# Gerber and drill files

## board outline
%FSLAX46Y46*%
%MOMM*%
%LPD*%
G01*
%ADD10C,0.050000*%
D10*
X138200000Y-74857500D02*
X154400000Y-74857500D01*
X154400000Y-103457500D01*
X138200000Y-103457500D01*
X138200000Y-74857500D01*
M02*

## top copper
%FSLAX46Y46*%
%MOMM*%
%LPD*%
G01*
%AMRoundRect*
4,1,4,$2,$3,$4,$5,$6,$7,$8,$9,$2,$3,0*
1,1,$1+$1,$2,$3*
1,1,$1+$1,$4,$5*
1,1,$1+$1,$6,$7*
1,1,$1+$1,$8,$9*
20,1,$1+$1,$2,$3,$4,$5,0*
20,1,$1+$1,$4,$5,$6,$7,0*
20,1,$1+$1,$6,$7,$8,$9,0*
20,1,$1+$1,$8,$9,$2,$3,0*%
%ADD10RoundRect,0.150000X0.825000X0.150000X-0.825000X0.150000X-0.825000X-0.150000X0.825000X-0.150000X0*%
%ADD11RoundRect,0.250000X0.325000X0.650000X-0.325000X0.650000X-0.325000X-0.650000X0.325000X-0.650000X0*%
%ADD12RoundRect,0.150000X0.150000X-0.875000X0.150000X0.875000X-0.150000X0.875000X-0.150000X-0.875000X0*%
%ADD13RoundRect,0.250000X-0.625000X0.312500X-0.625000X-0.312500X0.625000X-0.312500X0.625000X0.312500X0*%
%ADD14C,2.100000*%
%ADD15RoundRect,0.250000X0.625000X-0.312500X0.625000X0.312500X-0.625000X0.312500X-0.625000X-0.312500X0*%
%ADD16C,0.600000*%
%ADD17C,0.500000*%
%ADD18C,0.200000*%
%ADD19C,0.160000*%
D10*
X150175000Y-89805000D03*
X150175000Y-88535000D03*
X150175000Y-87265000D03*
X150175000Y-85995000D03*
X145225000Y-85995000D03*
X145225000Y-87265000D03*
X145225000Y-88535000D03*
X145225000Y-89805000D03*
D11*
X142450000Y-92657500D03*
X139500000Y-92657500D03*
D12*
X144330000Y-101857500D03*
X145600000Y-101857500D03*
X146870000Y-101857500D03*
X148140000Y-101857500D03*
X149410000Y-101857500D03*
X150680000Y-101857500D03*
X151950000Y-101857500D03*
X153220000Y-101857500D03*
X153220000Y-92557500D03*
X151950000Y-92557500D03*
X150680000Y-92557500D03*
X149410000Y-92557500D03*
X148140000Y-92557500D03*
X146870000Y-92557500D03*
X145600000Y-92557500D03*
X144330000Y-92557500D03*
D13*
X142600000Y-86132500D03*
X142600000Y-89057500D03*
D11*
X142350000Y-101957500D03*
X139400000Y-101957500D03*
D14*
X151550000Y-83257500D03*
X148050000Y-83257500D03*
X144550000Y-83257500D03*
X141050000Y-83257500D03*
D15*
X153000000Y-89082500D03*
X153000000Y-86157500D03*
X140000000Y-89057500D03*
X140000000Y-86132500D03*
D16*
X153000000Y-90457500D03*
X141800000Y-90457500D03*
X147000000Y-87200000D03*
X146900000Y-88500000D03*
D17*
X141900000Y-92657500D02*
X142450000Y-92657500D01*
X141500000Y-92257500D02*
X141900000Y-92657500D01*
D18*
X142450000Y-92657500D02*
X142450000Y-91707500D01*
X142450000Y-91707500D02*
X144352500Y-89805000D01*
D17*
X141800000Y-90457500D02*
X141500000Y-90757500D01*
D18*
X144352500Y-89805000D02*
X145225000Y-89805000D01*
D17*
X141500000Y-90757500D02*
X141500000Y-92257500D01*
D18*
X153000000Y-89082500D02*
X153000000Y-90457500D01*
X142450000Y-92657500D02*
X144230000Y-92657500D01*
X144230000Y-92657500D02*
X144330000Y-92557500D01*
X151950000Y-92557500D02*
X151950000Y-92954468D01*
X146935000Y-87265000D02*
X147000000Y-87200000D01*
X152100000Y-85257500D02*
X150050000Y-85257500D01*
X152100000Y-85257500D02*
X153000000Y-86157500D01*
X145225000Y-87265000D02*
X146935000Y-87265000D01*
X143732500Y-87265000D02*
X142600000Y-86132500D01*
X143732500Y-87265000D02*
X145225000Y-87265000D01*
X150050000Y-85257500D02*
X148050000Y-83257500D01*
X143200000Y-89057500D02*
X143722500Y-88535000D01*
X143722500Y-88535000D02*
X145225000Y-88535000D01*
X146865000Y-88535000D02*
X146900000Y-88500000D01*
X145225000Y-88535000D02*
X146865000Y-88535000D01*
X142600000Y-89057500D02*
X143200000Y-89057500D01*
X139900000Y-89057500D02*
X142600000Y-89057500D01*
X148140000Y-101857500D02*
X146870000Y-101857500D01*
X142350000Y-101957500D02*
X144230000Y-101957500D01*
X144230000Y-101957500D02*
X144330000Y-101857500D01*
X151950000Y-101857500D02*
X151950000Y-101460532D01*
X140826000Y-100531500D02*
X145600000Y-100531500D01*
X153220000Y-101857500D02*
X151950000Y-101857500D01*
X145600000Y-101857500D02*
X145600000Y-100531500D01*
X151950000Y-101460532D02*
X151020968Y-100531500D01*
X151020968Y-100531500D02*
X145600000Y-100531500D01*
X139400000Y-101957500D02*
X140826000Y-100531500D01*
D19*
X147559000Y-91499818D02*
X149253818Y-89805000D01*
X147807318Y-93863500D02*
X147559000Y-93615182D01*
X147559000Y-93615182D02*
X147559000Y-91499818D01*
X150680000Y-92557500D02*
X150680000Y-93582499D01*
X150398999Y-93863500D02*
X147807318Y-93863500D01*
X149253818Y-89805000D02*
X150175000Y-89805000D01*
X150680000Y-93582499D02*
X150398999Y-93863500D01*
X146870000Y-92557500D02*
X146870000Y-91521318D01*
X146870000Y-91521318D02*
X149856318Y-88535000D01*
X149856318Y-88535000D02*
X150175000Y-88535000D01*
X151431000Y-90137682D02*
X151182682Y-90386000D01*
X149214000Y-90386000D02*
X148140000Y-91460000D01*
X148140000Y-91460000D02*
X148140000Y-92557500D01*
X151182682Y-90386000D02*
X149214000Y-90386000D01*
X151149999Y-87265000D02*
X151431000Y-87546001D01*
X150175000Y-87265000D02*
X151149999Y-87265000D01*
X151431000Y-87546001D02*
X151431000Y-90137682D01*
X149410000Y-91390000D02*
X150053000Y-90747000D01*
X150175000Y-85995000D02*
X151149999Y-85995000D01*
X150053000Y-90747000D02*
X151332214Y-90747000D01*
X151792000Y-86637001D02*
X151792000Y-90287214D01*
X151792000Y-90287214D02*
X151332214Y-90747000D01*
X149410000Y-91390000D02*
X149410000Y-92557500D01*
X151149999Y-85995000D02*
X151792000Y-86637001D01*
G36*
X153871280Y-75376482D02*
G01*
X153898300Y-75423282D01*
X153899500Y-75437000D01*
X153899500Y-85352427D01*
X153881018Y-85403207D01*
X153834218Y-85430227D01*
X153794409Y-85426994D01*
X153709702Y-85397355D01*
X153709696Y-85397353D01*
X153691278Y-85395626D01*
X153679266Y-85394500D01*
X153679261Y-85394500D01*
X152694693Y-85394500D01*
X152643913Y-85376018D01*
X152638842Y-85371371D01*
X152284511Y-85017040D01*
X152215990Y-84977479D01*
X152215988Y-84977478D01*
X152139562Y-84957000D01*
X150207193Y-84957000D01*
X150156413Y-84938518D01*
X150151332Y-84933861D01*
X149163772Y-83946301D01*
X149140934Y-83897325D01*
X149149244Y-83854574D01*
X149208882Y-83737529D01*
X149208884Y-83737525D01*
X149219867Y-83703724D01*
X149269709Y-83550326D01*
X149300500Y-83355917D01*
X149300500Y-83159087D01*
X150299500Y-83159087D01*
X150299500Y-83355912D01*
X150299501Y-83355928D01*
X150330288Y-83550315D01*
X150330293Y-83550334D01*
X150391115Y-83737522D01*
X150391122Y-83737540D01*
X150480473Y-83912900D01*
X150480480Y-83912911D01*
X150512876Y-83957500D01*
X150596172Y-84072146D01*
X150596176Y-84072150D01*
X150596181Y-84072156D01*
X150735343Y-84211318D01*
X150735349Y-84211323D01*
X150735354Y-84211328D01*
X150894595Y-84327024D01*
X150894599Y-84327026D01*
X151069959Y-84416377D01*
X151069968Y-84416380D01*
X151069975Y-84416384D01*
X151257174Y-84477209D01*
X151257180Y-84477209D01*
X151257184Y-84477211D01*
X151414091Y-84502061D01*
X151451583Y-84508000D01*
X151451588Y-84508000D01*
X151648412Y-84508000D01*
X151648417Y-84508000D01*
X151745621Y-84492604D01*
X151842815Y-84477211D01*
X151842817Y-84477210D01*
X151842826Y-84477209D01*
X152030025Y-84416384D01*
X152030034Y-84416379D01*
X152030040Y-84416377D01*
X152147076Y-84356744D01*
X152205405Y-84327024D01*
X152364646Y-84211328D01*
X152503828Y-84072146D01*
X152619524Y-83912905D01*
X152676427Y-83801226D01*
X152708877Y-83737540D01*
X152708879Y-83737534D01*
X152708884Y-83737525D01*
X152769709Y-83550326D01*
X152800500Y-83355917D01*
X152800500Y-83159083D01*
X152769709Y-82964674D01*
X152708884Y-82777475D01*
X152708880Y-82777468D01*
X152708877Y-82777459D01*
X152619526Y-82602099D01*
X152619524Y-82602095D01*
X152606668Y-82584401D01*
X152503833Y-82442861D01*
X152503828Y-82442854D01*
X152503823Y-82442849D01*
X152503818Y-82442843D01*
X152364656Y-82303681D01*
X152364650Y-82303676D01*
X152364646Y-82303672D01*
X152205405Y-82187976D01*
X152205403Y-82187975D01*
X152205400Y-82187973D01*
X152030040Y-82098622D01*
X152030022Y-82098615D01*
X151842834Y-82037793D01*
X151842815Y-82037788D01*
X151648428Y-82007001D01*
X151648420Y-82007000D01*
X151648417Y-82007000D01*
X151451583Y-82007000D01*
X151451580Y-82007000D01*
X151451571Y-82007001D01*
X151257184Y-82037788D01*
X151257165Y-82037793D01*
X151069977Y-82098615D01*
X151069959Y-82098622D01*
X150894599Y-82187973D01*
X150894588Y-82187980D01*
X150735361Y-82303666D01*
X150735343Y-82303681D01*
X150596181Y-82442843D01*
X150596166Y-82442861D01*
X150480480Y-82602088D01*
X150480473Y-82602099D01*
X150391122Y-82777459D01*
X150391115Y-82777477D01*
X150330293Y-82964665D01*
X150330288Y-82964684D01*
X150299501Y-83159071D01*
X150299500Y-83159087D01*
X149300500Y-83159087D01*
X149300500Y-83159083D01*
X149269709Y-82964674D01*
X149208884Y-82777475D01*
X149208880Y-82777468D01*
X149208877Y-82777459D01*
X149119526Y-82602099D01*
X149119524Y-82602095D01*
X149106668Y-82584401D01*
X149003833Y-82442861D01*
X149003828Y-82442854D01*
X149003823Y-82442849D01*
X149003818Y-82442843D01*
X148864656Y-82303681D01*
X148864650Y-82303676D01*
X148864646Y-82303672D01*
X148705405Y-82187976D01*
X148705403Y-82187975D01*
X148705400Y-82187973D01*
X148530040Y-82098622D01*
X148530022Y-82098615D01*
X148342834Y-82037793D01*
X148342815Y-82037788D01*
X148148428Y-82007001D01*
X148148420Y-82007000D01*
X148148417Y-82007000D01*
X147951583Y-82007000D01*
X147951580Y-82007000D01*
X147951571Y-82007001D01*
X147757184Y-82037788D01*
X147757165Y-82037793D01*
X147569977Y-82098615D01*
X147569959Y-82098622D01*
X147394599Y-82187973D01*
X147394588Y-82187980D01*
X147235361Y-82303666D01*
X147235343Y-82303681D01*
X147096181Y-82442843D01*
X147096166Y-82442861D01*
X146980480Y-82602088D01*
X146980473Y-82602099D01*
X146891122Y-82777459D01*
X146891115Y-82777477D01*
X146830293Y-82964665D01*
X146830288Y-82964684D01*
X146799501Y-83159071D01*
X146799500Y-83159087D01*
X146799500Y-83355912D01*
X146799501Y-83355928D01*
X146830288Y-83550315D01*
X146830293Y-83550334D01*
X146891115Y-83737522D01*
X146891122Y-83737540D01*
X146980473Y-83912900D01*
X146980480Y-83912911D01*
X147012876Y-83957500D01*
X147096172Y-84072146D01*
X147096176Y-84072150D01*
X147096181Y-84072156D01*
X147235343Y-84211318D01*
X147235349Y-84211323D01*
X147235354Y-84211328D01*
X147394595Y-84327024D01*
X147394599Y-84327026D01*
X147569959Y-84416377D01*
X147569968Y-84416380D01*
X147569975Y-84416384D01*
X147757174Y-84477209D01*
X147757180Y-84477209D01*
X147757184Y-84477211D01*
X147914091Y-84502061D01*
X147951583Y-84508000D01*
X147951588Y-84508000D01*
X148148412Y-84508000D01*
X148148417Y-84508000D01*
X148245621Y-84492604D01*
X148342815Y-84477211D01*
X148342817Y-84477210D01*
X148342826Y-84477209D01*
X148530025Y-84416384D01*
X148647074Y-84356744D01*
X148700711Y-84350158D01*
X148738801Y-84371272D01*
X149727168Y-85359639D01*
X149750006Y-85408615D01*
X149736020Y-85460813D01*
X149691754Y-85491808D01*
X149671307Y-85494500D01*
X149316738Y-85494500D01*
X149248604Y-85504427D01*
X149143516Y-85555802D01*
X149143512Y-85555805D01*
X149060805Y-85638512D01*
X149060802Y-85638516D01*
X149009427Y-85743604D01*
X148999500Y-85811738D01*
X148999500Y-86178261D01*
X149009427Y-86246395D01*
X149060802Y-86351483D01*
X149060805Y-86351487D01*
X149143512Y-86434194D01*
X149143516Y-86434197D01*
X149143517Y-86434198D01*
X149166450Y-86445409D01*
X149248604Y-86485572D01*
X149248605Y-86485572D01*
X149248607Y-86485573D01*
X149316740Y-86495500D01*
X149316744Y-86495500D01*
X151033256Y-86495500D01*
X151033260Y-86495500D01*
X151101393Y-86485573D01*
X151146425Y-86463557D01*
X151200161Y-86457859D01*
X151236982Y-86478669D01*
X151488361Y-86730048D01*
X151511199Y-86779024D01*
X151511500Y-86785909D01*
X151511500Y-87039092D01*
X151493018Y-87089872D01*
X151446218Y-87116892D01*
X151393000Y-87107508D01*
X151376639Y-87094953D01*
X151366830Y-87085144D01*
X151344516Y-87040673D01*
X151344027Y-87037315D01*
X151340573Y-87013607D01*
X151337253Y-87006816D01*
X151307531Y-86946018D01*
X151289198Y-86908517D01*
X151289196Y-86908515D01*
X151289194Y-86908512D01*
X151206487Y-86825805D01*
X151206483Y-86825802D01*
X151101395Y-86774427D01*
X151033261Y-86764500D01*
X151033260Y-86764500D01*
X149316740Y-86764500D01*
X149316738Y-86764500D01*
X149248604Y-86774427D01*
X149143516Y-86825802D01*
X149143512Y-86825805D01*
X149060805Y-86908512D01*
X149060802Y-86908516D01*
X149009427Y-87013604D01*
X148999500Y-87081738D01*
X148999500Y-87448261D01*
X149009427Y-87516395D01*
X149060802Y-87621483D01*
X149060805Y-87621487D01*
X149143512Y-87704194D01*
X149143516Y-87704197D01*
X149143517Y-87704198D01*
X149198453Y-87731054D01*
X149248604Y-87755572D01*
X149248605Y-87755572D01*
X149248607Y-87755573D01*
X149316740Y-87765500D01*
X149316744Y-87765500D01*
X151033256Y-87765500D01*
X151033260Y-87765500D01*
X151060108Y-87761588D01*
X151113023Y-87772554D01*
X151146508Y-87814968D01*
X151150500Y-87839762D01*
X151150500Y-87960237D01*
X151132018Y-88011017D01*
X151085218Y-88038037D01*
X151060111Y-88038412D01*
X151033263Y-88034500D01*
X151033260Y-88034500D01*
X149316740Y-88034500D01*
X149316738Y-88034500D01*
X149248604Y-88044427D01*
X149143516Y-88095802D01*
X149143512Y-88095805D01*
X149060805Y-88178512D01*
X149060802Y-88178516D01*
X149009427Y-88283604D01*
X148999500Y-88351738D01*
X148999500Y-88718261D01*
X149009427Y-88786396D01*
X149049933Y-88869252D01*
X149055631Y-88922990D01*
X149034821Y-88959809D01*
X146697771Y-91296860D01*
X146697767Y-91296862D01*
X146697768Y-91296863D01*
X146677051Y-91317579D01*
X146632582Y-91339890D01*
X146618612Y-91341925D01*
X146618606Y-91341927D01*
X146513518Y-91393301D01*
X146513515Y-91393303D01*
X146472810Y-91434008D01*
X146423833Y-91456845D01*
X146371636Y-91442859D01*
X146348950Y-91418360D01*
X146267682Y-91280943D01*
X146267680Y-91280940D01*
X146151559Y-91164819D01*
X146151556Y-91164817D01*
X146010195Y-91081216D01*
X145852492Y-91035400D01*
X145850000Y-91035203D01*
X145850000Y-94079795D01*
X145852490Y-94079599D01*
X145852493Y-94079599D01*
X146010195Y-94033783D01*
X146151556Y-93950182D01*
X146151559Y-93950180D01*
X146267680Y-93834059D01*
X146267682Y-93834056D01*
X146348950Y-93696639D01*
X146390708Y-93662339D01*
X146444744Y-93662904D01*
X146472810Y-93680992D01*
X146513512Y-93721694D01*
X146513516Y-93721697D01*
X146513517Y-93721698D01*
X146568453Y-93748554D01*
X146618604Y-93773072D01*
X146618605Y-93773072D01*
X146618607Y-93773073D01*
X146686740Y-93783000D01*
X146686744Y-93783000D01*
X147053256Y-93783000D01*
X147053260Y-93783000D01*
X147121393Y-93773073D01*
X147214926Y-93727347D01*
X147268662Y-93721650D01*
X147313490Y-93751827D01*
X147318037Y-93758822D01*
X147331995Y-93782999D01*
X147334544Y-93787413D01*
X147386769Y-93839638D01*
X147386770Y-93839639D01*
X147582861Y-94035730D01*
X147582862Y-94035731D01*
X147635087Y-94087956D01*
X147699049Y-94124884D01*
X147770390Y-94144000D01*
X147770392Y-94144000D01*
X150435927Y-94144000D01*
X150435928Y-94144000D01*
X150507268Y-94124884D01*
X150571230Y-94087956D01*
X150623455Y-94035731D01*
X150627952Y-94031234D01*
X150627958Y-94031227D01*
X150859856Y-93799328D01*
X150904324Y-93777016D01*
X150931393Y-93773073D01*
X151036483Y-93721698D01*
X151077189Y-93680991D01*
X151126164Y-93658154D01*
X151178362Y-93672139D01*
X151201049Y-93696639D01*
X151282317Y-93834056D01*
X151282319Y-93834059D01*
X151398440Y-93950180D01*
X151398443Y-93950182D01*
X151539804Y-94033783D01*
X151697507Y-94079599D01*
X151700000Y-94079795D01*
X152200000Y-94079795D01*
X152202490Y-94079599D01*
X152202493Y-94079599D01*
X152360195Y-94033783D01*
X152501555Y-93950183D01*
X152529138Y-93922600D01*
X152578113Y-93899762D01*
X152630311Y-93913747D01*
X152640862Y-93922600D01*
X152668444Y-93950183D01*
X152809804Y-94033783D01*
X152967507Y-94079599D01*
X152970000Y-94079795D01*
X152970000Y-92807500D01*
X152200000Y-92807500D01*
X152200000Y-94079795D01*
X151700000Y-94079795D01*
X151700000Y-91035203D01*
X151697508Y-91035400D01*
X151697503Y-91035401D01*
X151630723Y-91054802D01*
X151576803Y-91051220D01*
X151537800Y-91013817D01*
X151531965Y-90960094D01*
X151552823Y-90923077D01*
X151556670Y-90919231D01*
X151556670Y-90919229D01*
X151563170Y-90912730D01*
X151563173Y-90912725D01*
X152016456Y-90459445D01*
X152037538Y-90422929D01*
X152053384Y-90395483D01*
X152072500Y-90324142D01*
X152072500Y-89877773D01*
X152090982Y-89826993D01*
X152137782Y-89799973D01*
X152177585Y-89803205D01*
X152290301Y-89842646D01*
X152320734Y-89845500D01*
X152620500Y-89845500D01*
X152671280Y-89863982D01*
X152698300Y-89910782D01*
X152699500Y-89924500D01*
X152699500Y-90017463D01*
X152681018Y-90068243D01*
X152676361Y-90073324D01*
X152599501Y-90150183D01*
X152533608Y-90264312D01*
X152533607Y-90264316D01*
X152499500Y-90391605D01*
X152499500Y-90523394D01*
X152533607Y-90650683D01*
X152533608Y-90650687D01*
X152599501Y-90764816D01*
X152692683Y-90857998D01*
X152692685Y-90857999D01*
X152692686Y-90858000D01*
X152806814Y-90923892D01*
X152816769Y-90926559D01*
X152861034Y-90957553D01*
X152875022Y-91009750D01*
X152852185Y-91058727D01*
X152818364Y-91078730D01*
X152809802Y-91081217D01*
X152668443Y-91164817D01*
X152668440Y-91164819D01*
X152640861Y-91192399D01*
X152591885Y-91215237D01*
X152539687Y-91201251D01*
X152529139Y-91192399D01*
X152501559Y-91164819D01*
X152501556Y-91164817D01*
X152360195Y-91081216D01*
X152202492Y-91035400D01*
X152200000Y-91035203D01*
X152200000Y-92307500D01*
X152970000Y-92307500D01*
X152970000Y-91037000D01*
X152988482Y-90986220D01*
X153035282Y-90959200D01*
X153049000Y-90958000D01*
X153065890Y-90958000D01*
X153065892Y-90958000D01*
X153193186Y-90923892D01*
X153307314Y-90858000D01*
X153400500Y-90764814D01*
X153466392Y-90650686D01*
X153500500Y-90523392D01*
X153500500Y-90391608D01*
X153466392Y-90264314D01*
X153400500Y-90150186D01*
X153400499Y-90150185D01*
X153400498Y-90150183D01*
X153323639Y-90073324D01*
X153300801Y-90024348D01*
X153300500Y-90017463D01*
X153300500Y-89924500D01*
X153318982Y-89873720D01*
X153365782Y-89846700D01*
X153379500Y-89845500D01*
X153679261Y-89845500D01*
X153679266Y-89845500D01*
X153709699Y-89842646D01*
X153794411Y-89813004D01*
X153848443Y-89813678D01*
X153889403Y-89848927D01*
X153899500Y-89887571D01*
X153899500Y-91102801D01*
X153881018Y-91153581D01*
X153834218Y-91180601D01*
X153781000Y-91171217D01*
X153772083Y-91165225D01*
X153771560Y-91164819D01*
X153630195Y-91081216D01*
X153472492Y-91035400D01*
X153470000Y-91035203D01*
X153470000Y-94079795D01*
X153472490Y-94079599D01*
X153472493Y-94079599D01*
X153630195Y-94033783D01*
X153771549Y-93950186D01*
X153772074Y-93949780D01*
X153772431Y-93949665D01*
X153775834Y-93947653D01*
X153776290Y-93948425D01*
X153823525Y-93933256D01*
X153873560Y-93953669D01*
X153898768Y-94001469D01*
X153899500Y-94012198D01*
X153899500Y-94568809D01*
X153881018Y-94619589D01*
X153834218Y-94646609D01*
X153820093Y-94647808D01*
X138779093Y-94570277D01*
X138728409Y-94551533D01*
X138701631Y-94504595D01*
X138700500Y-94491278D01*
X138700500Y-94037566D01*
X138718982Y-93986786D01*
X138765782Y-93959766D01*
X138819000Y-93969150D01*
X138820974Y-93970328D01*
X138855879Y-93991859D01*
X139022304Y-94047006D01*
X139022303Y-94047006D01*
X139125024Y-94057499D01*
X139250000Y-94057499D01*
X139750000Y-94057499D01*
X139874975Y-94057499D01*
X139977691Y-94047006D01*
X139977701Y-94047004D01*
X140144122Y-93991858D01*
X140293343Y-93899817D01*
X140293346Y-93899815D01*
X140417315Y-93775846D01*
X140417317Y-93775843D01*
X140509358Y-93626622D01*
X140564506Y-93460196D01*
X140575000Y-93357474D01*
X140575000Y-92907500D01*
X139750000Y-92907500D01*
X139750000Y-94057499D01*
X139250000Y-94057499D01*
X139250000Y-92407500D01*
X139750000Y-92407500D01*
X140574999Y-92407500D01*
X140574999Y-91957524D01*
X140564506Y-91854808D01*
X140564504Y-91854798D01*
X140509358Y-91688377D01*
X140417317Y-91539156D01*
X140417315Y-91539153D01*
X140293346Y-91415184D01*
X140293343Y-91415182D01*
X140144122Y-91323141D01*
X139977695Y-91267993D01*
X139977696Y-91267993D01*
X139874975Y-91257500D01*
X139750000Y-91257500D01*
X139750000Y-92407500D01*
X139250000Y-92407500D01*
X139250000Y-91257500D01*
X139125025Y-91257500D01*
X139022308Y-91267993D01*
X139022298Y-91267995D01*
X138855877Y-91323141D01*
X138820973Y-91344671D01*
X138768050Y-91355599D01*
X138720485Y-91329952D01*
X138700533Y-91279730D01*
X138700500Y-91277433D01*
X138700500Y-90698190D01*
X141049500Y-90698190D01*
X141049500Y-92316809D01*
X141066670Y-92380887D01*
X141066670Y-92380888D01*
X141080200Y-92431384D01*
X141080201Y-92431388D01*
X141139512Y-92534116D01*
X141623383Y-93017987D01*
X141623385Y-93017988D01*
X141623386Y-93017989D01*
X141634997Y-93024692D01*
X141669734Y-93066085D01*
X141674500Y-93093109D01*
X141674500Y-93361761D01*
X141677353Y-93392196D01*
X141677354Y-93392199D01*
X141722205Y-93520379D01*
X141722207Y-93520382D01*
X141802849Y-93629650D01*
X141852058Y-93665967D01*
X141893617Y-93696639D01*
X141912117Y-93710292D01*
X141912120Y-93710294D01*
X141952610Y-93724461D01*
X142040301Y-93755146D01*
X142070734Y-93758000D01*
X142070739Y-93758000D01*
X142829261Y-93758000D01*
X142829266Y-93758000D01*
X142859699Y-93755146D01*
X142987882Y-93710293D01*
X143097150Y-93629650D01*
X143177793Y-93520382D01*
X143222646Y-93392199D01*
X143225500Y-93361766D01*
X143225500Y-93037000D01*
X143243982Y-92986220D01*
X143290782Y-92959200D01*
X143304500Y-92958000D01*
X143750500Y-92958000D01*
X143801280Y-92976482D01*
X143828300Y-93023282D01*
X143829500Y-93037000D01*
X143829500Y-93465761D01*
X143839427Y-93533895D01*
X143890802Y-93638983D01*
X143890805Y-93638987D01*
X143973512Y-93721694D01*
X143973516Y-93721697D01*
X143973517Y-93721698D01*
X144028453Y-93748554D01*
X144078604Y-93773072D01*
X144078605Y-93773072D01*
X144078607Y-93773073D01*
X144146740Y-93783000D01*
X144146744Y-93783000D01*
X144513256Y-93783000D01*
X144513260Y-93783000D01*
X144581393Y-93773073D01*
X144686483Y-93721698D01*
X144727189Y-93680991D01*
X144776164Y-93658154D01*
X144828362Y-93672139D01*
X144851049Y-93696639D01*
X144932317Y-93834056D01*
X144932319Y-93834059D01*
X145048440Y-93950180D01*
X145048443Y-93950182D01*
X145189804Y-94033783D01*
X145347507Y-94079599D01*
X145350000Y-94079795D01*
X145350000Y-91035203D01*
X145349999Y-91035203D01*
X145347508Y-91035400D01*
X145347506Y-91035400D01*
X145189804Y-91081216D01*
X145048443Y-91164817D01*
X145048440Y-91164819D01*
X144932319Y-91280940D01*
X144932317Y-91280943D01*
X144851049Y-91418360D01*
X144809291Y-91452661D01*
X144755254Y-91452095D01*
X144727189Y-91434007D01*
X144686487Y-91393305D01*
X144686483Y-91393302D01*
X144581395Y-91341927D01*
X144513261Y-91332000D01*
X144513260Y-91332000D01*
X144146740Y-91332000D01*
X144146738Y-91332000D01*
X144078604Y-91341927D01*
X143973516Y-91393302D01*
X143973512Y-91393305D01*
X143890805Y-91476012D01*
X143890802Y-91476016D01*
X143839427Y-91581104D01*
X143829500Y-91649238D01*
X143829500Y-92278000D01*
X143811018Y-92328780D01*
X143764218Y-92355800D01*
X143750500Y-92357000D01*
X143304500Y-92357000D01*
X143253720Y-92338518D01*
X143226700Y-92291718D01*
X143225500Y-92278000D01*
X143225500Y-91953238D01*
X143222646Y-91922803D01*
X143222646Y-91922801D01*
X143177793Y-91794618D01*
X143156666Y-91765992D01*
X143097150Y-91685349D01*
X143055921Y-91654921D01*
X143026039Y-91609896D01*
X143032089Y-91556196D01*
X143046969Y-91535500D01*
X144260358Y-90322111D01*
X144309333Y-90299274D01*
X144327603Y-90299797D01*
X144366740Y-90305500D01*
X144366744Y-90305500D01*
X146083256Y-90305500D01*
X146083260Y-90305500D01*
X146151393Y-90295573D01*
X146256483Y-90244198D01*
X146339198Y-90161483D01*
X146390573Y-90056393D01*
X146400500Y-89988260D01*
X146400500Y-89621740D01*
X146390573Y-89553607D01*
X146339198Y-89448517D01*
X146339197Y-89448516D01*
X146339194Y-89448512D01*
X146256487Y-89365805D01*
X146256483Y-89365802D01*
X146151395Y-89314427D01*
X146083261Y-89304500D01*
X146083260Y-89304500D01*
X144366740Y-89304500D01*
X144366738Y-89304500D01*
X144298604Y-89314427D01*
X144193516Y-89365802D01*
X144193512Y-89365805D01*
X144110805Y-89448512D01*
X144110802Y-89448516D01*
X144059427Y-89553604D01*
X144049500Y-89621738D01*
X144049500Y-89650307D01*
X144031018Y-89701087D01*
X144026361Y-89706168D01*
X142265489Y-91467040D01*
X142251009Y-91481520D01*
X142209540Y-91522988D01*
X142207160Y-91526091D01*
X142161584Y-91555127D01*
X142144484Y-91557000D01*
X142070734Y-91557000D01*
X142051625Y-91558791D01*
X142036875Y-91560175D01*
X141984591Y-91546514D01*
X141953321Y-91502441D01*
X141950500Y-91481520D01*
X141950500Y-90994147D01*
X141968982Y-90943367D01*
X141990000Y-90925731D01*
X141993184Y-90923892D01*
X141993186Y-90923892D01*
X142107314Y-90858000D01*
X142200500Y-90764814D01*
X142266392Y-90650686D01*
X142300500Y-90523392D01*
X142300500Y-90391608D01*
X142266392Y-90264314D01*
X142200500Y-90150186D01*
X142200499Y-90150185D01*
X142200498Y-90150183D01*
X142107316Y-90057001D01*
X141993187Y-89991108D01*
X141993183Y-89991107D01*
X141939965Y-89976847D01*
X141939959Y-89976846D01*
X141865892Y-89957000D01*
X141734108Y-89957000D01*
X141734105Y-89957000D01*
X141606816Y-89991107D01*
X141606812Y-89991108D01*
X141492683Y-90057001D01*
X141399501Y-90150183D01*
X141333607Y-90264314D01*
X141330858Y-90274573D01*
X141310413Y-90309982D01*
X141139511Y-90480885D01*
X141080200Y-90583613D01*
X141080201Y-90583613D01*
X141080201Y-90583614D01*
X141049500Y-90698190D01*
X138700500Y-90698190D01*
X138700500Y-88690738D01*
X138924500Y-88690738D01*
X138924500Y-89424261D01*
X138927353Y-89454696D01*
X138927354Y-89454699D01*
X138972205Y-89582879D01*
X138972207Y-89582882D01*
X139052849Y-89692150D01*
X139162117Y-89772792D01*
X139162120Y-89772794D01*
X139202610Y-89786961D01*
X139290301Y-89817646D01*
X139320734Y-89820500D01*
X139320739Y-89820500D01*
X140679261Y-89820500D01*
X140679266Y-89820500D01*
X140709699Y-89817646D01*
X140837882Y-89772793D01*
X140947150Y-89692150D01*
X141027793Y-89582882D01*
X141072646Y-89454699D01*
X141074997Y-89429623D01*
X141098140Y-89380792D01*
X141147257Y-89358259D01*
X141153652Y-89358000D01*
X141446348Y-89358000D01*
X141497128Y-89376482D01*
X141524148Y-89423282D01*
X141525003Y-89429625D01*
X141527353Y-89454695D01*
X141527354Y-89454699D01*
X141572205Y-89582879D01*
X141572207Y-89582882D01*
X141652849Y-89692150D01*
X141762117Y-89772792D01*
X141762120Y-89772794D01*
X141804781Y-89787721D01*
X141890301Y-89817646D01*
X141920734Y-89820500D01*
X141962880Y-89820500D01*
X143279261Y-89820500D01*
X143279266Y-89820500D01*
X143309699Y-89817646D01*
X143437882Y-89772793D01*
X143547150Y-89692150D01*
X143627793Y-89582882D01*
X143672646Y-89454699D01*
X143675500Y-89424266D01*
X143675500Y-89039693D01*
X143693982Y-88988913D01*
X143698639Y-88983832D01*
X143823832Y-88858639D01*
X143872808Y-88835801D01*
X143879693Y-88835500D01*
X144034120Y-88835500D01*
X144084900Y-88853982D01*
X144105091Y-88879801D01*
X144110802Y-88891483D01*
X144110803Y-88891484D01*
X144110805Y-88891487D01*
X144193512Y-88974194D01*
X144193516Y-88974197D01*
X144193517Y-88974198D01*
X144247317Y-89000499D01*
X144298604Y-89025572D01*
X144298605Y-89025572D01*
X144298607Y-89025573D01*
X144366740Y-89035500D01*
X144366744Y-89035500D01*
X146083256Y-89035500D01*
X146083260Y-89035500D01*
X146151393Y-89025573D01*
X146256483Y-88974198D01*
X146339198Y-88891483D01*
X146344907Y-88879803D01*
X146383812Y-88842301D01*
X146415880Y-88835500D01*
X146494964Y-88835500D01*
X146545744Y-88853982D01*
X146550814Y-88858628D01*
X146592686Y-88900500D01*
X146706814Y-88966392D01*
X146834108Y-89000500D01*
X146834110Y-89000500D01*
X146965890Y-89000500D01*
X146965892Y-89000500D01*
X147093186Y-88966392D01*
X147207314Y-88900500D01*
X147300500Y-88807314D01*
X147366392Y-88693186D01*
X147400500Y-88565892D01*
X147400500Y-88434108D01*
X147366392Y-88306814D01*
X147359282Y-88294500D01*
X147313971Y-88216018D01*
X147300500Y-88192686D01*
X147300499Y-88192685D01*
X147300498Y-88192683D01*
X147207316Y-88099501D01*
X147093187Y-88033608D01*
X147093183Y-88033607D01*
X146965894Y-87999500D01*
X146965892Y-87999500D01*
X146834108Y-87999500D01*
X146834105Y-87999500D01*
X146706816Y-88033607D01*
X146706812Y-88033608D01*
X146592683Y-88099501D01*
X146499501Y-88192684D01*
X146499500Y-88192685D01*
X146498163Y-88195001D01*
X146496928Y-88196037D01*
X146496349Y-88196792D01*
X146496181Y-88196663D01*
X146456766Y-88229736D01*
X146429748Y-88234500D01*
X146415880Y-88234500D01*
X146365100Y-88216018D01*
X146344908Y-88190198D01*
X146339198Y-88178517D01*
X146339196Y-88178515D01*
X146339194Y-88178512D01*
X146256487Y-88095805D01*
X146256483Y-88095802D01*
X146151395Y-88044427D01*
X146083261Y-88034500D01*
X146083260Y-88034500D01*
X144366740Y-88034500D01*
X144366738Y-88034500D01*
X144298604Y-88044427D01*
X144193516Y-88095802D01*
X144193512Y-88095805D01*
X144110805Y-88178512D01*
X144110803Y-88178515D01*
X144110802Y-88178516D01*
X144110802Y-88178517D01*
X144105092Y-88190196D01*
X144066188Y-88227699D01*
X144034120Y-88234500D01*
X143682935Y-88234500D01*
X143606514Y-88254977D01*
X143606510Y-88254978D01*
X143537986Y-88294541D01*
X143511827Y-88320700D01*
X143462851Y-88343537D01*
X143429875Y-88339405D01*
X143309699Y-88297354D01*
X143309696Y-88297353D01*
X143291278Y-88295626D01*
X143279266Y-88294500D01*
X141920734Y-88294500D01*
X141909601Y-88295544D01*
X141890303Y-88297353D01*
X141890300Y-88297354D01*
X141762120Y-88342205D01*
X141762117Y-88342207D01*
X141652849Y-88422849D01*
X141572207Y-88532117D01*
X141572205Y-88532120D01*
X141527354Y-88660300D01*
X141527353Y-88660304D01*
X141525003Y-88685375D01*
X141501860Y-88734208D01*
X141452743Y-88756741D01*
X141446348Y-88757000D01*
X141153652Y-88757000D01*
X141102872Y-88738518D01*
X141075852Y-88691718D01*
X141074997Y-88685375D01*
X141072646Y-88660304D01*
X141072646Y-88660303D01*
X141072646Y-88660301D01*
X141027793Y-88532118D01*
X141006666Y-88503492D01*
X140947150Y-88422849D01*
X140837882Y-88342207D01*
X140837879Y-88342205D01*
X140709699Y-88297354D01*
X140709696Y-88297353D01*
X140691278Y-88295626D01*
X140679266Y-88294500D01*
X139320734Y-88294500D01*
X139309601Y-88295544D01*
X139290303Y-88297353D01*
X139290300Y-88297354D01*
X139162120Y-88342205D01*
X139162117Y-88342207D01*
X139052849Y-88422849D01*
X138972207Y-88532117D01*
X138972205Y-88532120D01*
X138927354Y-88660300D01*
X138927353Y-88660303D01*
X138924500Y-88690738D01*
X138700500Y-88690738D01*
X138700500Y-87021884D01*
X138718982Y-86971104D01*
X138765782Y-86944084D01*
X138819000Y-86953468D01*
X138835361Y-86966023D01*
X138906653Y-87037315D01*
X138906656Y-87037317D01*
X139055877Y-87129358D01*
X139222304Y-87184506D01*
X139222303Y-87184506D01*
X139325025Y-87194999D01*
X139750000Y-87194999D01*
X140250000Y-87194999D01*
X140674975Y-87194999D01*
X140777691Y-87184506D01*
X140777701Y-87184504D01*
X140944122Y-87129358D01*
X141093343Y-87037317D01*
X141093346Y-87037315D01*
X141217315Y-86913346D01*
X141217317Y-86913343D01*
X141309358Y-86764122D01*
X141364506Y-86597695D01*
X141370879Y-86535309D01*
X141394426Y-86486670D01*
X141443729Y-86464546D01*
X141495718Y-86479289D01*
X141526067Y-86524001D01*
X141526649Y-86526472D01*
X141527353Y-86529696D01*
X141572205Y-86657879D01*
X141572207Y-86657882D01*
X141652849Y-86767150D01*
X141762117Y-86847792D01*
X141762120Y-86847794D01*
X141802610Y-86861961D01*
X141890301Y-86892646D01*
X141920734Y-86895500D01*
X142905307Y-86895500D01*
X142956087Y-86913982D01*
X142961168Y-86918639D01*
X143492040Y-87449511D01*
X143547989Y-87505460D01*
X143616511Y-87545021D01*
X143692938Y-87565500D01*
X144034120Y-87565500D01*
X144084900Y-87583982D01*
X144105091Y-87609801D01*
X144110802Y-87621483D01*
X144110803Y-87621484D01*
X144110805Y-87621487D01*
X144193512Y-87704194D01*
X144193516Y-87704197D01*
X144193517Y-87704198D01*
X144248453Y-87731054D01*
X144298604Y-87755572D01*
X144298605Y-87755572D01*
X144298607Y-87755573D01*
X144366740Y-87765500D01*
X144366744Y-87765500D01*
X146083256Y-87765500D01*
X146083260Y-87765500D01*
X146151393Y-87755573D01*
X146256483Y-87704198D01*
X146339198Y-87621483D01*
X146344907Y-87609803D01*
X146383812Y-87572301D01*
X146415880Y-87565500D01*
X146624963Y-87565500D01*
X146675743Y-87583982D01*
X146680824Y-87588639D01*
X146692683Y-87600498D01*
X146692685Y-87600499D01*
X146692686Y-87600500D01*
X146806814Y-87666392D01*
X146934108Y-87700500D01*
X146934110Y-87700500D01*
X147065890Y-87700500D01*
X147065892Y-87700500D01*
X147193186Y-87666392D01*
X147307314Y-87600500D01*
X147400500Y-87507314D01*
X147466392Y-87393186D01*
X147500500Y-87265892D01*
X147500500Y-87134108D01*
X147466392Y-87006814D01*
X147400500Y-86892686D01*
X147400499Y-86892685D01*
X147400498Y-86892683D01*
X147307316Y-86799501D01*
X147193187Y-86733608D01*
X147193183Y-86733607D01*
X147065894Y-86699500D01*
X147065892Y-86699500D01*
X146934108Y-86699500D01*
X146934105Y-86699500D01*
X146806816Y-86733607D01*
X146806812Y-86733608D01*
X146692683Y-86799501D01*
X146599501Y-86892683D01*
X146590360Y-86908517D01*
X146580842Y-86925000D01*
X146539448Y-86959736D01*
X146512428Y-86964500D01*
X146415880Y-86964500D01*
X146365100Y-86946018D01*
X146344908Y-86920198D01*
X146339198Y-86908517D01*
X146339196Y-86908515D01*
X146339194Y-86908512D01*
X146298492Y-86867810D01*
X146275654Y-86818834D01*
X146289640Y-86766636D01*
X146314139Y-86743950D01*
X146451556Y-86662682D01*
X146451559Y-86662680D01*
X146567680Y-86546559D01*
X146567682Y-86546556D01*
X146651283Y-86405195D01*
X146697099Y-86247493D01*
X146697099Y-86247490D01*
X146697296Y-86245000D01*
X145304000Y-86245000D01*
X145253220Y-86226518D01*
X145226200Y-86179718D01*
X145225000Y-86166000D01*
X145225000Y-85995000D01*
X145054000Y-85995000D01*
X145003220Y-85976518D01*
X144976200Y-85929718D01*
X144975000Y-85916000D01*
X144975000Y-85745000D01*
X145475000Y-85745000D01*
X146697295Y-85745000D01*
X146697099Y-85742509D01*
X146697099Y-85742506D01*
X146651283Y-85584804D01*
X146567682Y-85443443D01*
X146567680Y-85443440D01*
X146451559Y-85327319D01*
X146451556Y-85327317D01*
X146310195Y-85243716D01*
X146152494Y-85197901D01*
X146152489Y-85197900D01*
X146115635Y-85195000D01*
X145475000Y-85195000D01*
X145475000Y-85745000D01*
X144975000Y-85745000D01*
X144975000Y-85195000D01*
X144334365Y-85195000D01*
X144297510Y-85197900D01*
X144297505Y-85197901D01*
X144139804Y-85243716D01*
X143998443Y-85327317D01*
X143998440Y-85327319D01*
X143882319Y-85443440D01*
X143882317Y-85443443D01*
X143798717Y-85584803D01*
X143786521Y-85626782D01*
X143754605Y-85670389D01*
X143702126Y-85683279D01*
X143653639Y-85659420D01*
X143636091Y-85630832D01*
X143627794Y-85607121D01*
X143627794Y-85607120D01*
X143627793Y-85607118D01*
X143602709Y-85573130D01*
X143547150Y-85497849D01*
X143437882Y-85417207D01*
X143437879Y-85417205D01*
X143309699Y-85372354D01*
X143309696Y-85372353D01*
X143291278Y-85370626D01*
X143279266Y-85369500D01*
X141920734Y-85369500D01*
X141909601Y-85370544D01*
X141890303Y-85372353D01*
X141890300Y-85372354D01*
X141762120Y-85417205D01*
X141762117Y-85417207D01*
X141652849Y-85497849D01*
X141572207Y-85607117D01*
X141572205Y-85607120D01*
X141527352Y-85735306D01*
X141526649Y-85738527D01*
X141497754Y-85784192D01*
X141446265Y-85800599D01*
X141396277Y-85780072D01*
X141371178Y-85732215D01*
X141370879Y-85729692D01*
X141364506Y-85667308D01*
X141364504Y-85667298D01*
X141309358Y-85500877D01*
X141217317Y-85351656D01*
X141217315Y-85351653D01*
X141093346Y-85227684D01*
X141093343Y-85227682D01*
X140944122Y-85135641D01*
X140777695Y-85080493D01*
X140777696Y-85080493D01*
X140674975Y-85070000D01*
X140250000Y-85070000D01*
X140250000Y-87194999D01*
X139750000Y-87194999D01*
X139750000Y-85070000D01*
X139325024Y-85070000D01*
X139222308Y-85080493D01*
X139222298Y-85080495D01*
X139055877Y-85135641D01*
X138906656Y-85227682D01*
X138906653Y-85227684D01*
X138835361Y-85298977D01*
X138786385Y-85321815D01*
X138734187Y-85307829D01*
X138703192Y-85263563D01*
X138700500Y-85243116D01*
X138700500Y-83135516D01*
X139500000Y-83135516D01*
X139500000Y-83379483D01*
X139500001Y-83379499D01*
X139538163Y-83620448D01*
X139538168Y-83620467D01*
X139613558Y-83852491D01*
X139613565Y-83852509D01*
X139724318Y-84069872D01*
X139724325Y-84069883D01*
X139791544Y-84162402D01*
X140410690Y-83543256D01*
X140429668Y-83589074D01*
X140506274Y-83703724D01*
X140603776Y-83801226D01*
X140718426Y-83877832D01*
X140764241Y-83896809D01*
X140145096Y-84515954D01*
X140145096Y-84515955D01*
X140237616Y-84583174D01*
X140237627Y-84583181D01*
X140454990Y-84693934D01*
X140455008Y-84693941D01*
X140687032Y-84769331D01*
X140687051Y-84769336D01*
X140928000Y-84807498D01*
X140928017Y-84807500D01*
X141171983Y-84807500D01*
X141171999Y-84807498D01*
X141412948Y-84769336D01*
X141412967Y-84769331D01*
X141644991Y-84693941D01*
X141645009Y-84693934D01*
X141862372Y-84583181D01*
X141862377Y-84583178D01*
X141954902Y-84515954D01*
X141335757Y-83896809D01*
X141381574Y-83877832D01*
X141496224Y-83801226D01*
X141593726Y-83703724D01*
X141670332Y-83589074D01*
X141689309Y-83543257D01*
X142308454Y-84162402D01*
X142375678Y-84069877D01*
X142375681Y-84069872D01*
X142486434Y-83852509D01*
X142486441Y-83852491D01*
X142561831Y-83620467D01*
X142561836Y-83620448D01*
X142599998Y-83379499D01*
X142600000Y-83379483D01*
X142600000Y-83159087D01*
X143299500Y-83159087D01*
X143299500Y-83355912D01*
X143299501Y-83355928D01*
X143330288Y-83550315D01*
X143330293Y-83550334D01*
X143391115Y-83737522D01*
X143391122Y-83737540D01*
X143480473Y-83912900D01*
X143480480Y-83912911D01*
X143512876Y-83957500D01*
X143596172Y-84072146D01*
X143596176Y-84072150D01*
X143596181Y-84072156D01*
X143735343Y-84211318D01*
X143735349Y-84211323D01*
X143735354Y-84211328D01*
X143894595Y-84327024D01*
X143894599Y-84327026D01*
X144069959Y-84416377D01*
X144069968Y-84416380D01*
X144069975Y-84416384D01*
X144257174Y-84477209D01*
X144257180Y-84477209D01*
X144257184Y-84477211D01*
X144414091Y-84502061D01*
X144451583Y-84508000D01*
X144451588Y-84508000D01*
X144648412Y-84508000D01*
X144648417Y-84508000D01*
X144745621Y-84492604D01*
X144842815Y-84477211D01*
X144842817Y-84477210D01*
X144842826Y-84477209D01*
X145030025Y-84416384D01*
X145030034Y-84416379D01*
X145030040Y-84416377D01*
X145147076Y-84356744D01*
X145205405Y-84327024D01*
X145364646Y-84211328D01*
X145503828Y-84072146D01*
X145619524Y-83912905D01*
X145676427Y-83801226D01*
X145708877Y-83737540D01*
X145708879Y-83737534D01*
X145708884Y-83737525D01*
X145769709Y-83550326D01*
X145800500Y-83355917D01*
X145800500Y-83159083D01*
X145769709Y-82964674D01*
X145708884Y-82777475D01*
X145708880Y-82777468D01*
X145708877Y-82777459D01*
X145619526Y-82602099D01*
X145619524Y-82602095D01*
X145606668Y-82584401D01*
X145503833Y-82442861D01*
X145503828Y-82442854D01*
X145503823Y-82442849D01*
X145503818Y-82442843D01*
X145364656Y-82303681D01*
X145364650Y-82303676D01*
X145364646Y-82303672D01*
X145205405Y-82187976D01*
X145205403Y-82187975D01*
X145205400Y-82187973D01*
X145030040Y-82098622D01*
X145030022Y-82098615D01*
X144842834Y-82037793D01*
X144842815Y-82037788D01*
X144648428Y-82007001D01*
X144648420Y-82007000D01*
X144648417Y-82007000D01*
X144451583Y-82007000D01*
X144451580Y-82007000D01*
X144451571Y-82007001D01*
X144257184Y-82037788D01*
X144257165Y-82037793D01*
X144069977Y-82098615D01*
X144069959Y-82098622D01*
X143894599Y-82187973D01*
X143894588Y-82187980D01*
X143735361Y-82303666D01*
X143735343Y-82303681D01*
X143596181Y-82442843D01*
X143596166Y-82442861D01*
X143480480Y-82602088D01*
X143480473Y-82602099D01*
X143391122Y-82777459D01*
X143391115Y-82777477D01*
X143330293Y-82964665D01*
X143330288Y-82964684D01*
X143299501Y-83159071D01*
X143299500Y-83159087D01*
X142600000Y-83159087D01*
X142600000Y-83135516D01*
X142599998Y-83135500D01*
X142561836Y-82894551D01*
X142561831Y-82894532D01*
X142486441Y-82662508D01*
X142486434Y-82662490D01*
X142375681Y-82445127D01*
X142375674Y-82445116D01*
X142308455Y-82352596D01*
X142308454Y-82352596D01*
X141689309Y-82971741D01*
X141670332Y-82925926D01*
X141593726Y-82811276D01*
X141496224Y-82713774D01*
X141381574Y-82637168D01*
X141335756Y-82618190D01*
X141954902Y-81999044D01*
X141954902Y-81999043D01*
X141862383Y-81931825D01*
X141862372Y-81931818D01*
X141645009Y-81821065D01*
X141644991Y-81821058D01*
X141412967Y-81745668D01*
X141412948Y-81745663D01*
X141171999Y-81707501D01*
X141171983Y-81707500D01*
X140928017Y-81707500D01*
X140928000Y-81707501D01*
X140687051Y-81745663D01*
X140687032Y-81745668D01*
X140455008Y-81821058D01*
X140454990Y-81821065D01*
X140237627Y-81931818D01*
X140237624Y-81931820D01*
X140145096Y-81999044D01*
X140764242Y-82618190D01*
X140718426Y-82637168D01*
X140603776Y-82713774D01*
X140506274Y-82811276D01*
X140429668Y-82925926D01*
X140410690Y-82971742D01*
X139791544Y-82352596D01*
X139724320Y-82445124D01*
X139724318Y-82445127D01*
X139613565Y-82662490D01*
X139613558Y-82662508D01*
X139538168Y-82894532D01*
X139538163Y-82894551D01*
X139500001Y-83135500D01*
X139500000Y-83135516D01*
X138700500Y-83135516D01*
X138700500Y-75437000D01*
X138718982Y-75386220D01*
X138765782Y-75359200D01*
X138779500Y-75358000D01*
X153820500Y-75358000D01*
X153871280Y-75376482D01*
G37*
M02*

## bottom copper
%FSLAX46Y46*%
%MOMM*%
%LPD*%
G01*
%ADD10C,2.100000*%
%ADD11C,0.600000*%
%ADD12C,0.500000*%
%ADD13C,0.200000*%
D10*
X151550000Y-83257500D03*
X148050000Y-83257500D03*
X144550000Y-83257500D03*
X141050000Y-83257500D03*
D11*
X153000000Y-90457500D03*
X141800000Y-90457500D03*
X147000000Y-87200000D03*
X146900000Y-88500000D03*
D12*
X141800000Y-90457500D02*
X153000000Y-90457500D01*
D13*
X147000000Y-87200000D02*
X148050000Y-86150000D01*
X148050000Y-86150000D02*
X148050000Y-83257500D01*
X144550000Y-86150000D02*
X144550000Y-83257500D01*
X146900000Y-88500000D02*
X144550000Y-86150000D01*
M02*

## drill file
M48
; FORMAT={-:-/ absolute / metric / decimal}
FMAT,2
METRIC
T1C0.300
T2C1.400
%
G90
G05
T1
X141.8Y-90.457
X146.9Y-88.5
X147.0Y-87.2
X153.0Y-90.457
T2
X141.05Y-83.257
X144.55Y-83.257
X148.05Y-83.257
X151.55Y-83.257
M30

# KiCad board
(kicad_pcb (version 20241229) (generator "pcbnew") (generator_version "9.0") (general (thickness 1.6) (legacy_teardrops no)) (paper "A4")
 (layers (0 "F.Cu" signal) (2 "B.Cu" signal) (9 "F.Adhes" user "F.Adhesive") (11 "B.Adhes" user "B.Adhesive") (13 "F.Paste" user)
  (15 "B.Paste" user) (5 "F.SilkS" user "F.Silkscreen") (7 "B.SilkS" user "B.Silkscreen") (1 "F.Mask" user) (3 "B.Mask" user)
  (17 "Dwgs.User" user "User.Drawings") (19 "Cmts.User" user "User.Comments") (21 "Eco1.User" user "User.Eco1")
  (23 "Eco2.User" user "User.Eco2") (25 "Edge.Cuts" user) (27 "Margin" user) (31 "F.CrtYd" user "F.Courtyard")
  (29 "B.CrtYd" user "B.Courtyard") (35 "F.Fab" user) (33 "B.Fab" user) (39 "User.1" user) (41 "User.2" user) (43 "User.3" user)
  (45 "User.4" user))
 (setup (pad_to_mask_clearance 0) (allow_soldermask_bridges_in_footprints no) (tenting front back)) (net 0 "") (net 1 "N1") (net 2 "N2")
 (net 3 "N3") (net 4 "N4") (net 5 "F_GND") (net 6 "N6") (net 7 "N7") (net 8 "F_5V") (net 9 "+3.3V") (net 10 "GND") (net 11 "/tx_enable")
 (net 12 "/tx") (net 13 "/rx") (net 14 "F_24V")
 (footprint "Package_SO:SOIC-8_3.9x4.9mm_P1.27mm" (layer "F.Cu") (at 147.7 87.9 180)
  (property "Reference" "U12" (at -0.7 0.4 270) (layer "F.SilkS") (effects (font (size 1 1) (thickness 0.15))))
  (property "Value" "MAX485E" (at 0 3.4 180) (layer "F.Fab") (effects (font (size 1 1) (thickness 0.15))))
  (pad "1" smd roundrect (at -2.475 -1.905 180) (size 1.95 0.6) (layers "F.Cu" "F.Mask" "F.Paste") (roundrect_rratio 0.25) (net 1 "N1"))
  (pad "2" smd roundrect (at -2.475 -0.635 180) (size 1.95 0.6) (layers "F.Cu" "F.Mask" "F.Paste") (roundrect_rratio 0.25) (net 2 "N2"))
  (pad "3" smd roundrect (at -2.475 0.635 180) (size 1.95 0.6) (layers "F.Cu" "F.Mask" "F.Paste") (roundrect_rratio 0.25) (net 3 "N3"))
  (pad "4" smd roundrect (at -2.475 1.905 180) (size 1.95 0.6) (layers "F.Cu" "F.Mask" "F.Paste") (roundrect_rratio 0.25) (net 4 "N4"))
  (pad "5" smd roundrect (at 2.475 1.905 180) (size 1.95 0.6) (layers "F.Cu" "F.Mask" "F.Paste") (roundrect_rratio 0.25) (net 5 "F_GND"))
  (pad "6" smd roundrect (at 2.475 0.635 180) (size 1.95 0.6) (layers "F.Cu" "F.Mask" "F.Paste") (roundrect_rratio 0.25) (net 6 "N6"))
  (pad "7" smd roundrect (at 2.475 -0.635 180) (size 1.95 0.6) (layers "F.Cu" "F.Mask" "F.Paste") (roundrect_rratio 0.25) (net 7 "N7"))
  (pad "8" smd roundrect (at 2.475 -1.905 180) (size 1.95 0.6) (layers "F.Cu" "F.Mask" "F.Paste") (roundrect_rratio 0.25) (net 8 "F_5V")))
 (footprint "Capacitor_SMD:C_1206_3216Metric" (layer "F.Cu") (at 140.975 92.6575 180)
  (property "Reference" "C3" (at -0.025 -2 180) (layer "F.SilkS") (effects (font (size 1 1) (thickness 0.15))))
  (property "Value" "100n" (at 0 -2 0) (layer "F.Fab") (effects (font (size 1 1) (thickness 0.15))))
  (pad "1" smd roundrect (at -1.475 0 180) (size 1.15 1.8) (layers "F.Cu" "F.Mask" "F.Paste") (roundrect_rratio 0.217391) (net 8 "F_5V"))
  (pad "2" smd roundrect (at 1.475 0 180) (size 1.15 1.8) (layers "F.Cu" "F.Mask" "F.Paste") (roundrect_rratio 0.217391) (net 5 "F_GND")))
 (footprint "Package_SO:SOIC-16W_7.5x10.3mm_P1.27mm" (layer "F.Cu") (at 148.775 97.2075 90)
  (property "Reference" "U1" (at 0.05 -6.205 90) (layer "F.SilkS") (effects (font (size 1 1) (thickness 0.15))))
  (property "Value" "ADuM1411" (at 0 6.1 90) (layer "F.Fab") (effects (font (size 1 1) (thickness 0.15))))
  (pad "1" smd roundrect (at -4.65 -4.445 90) (size 2.05 0.6) (layers "F.Cu" "F.Mask" "F.Paste") (roundrect_rratio 0.25) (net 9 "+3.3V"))
  (pad "2" smd roundrect (at -4.65 -3.175 90) (size 2.05 0.6) (layers "F.Cu" "F.Mask" "F.Paste") (roundrect_rratio 0.25) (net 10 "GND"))
  (pad "3" smd roundrect (at -4.65 -1.905 90) (size 2.05 0.6) (layers "F.Cu" "F.Mask" "F.Paste") (roundrect_rratio 0.25)
   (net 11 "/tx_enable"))
  (pad "4" smd roundrect (at -4.65 -0.635 90) (size 2.05 0.6) (layers "F.Cu" "F.Mask" "F.Paste") (roundrect_rratio 0.25)
   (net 11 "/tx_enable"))
  (pad "5" smd roundrect (at -4.65 0.635 90) (size 2.05 0.6) (layers "F.Cu" "F.Mask" "F.Paste") (roundrect_rratio 0.25) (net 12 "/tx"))
  (pad "6" smd roundrect (at -4.65 1.905 90) (size 2.05 0.6) (layers "F.Cu" "F.Mask" "F.Paste") (roundrect_rratio 0.25) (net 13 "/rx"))
  (pad "7" smd roundrect (at -4.65 3.175 90) (size 2.05 0.6) (layers "F.Cu" "F.Mask" "F.Paste") (roundrect_rratio 0.25) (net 10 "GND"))
  (pad "8" smd roundrect (at -4.65 4.445 90) (size 2.05 0.6) (layers "F.Cu" "F.Mask" "F.Paste") (roundrect_rratio 0.25) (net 10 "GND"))
  (pad "9" smd roundrect (at 4.65 4.445 90) (size 2.05 0.6) (layers "F.Cu" "F.Mask" "F.Paste") (roundrect_rratio 0.25) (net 5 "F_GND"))
  (pad "10" smd roundrect (at 4.65 3.175 90) (size 2.05 0.6) (layers "F.Cu" "F.Mask" "F.Paste") (roundrect_rratio 0.25) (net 5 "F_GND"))
  (pad "11" smd roundrect (at 4.65 1.905 90) (size 2.05 0.6) (layers "F.Cu" "F.Mask" "F.Paste") (roundrect_rratio 0.25) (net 1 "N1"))
  (pad "12" smd roundrect (at 4.65 0.635 90) (size 2.05 0.6) (layers "F.Cu" "F.Mask" "F.Paste") (roundrect_rratio 0.25) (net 4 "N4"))
  (pad "13" smd roundrect (at 4.65 -0.635 90) (size 2.05 0.6) (layers "F.Cu" "F.Mask" "F.Paste") (roundrect_rratio 0.25) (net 3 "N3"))
  (pad "14" smd roundrect (at 4.65 -1.905 90) (size 2.05 0.6) (layers "F.Cu" "F.Mask" "F.Paste") (roundrect_rratio 0.25) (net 2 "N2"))
  (pad "15" smd roundrect (at 4.65 -3.175 90) (size 2.05 0.6) (layers "F.Cu" "F.Mask" "F.Paste") (roundrect_rratio 0.25) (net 5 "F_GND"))
  (pad "16" smd roundrect (at 4.65 -4.445 90) (size 2.05 0.6) (layers "F.Cu" "F.Mask" "F.Paste") (roundrect_rratio 0.25) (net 8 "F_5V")))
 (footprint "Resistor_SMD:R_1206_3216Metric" (layer "F.Cu") (at 142.6 87.595 -90)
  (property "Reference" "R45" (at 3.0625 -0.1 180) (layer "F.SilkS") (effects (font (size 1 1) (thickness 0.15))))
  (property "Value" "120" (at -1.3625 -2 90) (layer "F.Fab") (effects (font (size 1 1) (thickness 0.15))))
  (pad "1" smd roundrect (at -1.4625 0 270) (size 1.125 1.75) (layers "F.Cu" "F.Mask" "F.Paste") (roundrect_rratio 0.222222) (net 6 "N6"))
  (pad "2" smd roundrect (at 1.4625 0 270) (size 1.125 1.75) (layers "F.Cu" "F.Mask" "F.Paste") (roundrect_rratio 0.222222) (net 7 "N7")))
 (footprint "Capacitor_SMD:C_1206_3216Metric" (layer "F.Cu") (at 140.875 101.9575 180)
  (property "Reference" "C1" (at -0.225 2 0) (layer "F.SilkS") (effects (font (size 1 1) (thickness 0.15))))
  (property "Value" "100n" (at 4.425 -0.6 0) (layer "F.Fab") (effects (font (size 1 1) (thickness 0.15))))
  (pad "1" smd roundrect (at -1.475 0 180) (size 1.15 1.8) (layers "F.Cu" "F.Mask" "F.Paste") (roundrect_rratio 0.217391) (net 9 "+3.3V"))
  (pad "2" smd roundrect (at 1.475 0 180) (size 1.15 1.8) (layers "F.Cu" "F.Mask" "F.Paste") (roundrect_rratio 0.217391) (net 10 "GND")))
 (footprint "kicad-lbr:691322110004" (layer "F.Cu") (at 146.3 83.2575 180)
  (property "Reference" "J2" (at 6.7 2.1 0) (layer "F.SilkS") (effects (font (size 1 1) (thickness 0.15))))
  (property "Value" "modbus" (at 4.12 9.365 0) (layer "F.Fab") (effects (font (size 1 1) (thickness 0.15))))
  (pad "1" thru_hole circle (at -5.25 0 180) (size 2.1 2.1) (drill 1.4) (layers "*.Cu" "*.Mask") (remove_unused_layers no) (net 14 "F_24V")
   (solder_mask_margin 0.102))
  (pad "2" thru_hole circle (at -1.75 0 180) (size 2.1 2.1) (drill 1.4) (layers "*.Cu" "*.Mask") (remove_unused_layers no) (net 6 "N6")
   (solder_mask_margin 0.102))
  (pad "3" thru_hole circle (at 1.75 0 180) (size 2.1 2.1) (drill 1.4) (layers "*.Cu" "*.Mask") (remove_unused_layers no) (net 7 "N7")
   (solder_mask_margin 0.102))
  (pad "4" thru_hole circle (at 5.25 0 180) (size 2.1 2.1) (drill 1.4) (layers "*.Cu" "*.Mask") (remove_unused_layers no) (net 5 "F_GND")
   (solder_mask_margin 0.102)))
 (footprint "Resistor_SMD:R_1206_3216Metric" (layer "F.Cu") (at 153 87.62 90)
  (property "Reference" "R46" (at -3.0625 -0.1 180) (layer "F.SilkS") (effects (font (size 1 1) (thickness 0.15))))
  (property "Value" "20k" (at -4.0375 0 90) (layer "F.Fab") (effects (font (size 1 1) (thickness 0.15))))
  (pad "1" smd roundrect (at -1.4625 0 90) (size 1.125 1.75) (layers "F.Cu" "F.Mask" "F.Paste") (roundrect_rratio 0.222222) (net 8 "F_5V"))
  (pad "2" smd roundrect (at 1.4625 0 90) (size 1.125 1.75) (layers "F.Cu" "F.Mask" "F.Paste") (roundrect_rratio 0.222222) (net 6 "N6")))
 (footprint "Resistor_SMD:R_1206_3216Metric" (layer "F.Cu") (at 140 87.595 90)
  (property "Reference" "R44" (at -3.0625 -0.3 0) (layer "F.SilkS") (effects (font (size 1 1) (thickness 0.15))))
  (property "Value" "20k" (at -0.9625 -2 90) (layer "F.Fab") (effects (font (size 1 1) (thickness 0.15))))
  (pad "1" smd roundrect (at -1.4625 0 90) (size 1.125 1.75) (layers "F.Cu" "F.Mask" "F.Paste") (roundrect_rratio 0.222222) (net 7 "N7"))
  (pad "2" smd roundrect (at 1.4625 0 90) (size 1.125 1.75) (layers "F.Cu" "F.Mask" "F.Paste") (roundrect_rratio 0.222222) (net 5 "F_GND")))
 (gr_rect (start 138.2 74.8575) (end 154.4 103.4575) (stroke (width 0.05) (type default)) (fill no) (layer "Edge.Cuts"))
 (segment (start 141.9 92.6575) (end 142.45 92.6575) (width 0.5) (layer "F.Cu") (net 8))
 (segment (start 141.5 92.2575) (end 141.9 92.6575) (width 0.5) (layer "F.Cu") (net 8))
 (segment (start 142.45 92.6575) (end 142.45 91.7075) (width 0.2) (layer "F.Cu") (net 8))
 (segment (start 142.45 91.7075) (end 144.3525 89.805) (width 0.2) (layer "F.Cu") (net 8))
 (segment (start 141.8 90.4575) (end 141.5 90.7575) (width 0.5) (layer "F.Cu") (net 8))
 (segment (start 144.3525 89.805) (end 145.225 89.805) (width 0.2) (layer "F.Cu") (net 8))
 (segment (start 141.5 90.7575) (end 141.5 92.2575) (width 0.5) (layer "F.Cu") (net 8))
 (segment (start 153 89.0825) (end 153 90.4575) (width 0.2) (layer "F.Cu") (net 8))
 (segment (start 142.45 92.6575) (end 144.23 92.6575) (width 0.2) (layer "F.Cu") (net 8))
 (segment (start 144.23 92.6575) (end 144.33 92.5575) (width 0.2) (layer "F.Cu") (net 8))
 (via (at 153 90.4575) (size 0.6) (drill 0.3) (layers "F.Cu" "B.Cu") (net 8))
 (via (at 141.8 90.4575) (size 0.6) (drill 0.3) (layers "F.Cu" "B.Cu") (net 8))
 (segment (start 141.8 90.4575) (end 153 90.4575) (width 0.5) (layer "B.Cu") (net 8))
 (segment (start 151.95 92.5575) (end 151.95 92.954468) (width 0.2) (layer "F.Cu") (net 5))
 (segment (start 146.935 87.265) (end 147 87.2) (width 0.2) (layer "F.Cu") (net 6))
 (segment (start 152.1 85.2575) (end 150.05 85.2575) (width 0.2) (layer "F.Cu") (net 6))
 (segment (start 152.1 85.2575) (end 153 86.1575) (width 0.2) (layer "F.Cu") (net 6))
 (segment (start 145.225 87.265) (end 146.935 87.265) (width 0.2) (layer "F.Cu") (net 6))
 (segment (start 143.7325 87.265) (end 142.6 86.1325) (width 0.2) (layer "F.Cu") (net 6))
 (segment (start 143.7325 87.265) (end 145.225 87.265) (width 0.2) (layer "F.Cu") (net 6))
 (segment (start 150.05 85.2575) (end 148.05 83.2575) (width 0.2) (layer "F.Cu") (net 6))
 (via (at 147 87.2) (size 0.6) (drill 0.3) (layers "F.Cu" "B.Cu") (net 6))
 (segment (start 147 87.2) (end 148.05 86.15) (width 0.2) (layer "B.Cu") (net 6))
 (segment (start 148.05 86.15) (end 148.05 83.2575) (width 0.2) (layer "B.Cu") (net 6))
 (segment (start 143.2 89.0575) (end 143.7225 88.535) (width 0.2) (layer "F.Cu") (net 7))
 (segment (start 143.7225 88.535) (end 145.225 88.535) (width 0.2) (layer "F.Cu") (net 7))
 (segment (start 146.865 88.535) (end 146.9 88.5) (width 0.2) (layer "F.Cu") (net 7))
 (segment (start 145.225 88.535) (end 146.865 88.535) (width 0.2) (layer "F.Cu") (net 7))
 (segment (start 142.6 89.0575) (end 143.2 89.0575) (width 0.2) (layer "F.Cu") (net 7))
 (segment (start 139.9 89.0575) (end 142.6 89.0575) (width 0.2) (layer "F.Cu") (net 7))
 (via (at 146.9 88.5) (size 0.6) (drill 0.3) (layers "F.Cu" "B.Cu") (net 7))
 (segment (start 144.55 86.15) (end 144.55 83.2575) (width 0.2) (layer "B.Cu") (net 7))
 (segment (start 146.9 88.5) (end 144.55 86.15) (width 0.2) (layer "B.Cu") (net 7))
 (segment (start 148.14 101.8575) (end 146.87 101.8575) (width 0.2) (layer "F.Cu") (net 11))
 (segment (start 142.35 101.9575) (end 144.23 101.9575) (width 0.2) (layer "F.Cu") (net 9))
 (segment (start 144.23 101.9575) (end 144.33 101.8575) (width 0.2) (layer "F.Cu") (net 9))
 (segment (start 151.95 101.8575) (end 151.95 101.460532) (width 0.2) (layer "F.Cu") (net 10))
 (segment (start 140.826 100.5315) (end 145.6 100.5315) (width 0.2) (layer "F.Cu") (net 10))
 (segment (start 153.22 101.8575) (end 151.95 101.8575) (width 0.2) (layer "F.Cu") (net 10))
 (segment (start 145.6 101.8575) (end 145.6 100.5315) (width 0.2) (layer "F.Cu") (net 10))
 (segment (start 151.95 101.460532) (end 151.020968 100.5315) (width 0.2) (layer "F.Cu") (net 10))
 (segment (start 151.020968 100.5315) (end 145.6 100.5315) (width 0.2) (layer "F.Cu") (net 10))
 (segment (start 139.4 101.9575) (end 140.826 100.5315) (width 0.2) (layer "F.Cu") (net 10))
 (segment (start 147.559 91.499818) (end 149.253818 89.805) (width 0.16) (layer "F.Cu") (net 1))
 (segment (start 147.807318 93.8635) (end 147.559 93.615182) (width 0.16) (layer "F.Cu") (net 1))
 (segment (start 147.559 93.615182) (end 147.559 91.499818) (width 0.16) (layer "F.Cu") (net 1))
 (segment (start 150.68 92.5575) (end 150.68 93.582499) (width 0.16) (layer "F.Cu") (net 1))
 (segment (start 150.398999 93.8635) (end 147.807318 93.8635) (width 0.16) (layer "F.Cu") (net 1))
 (segment (start 149.253818 89.805) (end 150.175 89.805) (width 0.16) (layer "F.Cu") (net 1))
 (segment (start 150.68 93.582499) (end 150.398999 93.8635) (width 0.16) (layer "F.Cu") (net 1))
 (segment (start 146.87 92.5575) (end 146.87 91.521318) (width 0.16) (layer "F.Cu") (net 2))
 (segment (start 146.87 91.521318) (end 149.856318 88.535) (width 0.16) (layer "F.Cu") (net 2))
 (segment (start 149.856318 88.535) (end 150.175 88.535) (width 0.16) (layer "F.Cu") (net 2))
 (segment (start 151.431 90.137682) (end 151.182682 90.386) (width 0.16) (layer "F.Cu") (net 3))
 (segment (start 149.214 90.386) (end 148.14 91.46) (width 0.16) (layer "F.Cu") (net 3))
 (segment (start 148.14 91.46) (end 148.14 92.5575) (width 0.16) (layer "F.Cu") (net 3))
 (segment (start 151.182682 90.386) (end 149.214 90.386) (width 0.16) (layer "F.Cu") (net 3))
 (segment (start 151.149999 87.265) (end 151.431 87.546001) (width 0.16) (layer "F.Cu") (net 3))
 (segment (start 150.175 87.265) (end 151.149999 87.265) (width 0.16) (layer "F.Cu") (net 3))
 (segment (start 151.431 87.546001) (end 151.431 90.137682) (width 0.16) (layer "F.Cu") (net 3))
 (segment (start 149.41 91.39) (end 150.053 90.747) (width 0.16) (layer "F.Cu") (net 4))
 (segment (start 150.175 85.995) (end 151.149999 85.995) (width 0.16) (layer "F.Cu") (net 4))
 (segment (start 150.053 90.747) (end 151.332214 90.747) (width 0.16) (layer "F.Cu") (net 4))
 (segment (start 151.792 86.637001) (end 151.792 90.287214) (width 0.16) (layer "F.Cu") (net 4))
 (segment (start 151.792 90.287214) (end 151.332214 90.747) (width 0.16) (layer "F.Cu") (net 4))
 (segment (start 149.41 91.39) (end 149.41 92.5575) (width 0.16) (layer "F.Cu") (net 4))
 (segment (start 151.149999 85.995) (end 151.792 86.637001) (width 0.16) (layer "F.Cu") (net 4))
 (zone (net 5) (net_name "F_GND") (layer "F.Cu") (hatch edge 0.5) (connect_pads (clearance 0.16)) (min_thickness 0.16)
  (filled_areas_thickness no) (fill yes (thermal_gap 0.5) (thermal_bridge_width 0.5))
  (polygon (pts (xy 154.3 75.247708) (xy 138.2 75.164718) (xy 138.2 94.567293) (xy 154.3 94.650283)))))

